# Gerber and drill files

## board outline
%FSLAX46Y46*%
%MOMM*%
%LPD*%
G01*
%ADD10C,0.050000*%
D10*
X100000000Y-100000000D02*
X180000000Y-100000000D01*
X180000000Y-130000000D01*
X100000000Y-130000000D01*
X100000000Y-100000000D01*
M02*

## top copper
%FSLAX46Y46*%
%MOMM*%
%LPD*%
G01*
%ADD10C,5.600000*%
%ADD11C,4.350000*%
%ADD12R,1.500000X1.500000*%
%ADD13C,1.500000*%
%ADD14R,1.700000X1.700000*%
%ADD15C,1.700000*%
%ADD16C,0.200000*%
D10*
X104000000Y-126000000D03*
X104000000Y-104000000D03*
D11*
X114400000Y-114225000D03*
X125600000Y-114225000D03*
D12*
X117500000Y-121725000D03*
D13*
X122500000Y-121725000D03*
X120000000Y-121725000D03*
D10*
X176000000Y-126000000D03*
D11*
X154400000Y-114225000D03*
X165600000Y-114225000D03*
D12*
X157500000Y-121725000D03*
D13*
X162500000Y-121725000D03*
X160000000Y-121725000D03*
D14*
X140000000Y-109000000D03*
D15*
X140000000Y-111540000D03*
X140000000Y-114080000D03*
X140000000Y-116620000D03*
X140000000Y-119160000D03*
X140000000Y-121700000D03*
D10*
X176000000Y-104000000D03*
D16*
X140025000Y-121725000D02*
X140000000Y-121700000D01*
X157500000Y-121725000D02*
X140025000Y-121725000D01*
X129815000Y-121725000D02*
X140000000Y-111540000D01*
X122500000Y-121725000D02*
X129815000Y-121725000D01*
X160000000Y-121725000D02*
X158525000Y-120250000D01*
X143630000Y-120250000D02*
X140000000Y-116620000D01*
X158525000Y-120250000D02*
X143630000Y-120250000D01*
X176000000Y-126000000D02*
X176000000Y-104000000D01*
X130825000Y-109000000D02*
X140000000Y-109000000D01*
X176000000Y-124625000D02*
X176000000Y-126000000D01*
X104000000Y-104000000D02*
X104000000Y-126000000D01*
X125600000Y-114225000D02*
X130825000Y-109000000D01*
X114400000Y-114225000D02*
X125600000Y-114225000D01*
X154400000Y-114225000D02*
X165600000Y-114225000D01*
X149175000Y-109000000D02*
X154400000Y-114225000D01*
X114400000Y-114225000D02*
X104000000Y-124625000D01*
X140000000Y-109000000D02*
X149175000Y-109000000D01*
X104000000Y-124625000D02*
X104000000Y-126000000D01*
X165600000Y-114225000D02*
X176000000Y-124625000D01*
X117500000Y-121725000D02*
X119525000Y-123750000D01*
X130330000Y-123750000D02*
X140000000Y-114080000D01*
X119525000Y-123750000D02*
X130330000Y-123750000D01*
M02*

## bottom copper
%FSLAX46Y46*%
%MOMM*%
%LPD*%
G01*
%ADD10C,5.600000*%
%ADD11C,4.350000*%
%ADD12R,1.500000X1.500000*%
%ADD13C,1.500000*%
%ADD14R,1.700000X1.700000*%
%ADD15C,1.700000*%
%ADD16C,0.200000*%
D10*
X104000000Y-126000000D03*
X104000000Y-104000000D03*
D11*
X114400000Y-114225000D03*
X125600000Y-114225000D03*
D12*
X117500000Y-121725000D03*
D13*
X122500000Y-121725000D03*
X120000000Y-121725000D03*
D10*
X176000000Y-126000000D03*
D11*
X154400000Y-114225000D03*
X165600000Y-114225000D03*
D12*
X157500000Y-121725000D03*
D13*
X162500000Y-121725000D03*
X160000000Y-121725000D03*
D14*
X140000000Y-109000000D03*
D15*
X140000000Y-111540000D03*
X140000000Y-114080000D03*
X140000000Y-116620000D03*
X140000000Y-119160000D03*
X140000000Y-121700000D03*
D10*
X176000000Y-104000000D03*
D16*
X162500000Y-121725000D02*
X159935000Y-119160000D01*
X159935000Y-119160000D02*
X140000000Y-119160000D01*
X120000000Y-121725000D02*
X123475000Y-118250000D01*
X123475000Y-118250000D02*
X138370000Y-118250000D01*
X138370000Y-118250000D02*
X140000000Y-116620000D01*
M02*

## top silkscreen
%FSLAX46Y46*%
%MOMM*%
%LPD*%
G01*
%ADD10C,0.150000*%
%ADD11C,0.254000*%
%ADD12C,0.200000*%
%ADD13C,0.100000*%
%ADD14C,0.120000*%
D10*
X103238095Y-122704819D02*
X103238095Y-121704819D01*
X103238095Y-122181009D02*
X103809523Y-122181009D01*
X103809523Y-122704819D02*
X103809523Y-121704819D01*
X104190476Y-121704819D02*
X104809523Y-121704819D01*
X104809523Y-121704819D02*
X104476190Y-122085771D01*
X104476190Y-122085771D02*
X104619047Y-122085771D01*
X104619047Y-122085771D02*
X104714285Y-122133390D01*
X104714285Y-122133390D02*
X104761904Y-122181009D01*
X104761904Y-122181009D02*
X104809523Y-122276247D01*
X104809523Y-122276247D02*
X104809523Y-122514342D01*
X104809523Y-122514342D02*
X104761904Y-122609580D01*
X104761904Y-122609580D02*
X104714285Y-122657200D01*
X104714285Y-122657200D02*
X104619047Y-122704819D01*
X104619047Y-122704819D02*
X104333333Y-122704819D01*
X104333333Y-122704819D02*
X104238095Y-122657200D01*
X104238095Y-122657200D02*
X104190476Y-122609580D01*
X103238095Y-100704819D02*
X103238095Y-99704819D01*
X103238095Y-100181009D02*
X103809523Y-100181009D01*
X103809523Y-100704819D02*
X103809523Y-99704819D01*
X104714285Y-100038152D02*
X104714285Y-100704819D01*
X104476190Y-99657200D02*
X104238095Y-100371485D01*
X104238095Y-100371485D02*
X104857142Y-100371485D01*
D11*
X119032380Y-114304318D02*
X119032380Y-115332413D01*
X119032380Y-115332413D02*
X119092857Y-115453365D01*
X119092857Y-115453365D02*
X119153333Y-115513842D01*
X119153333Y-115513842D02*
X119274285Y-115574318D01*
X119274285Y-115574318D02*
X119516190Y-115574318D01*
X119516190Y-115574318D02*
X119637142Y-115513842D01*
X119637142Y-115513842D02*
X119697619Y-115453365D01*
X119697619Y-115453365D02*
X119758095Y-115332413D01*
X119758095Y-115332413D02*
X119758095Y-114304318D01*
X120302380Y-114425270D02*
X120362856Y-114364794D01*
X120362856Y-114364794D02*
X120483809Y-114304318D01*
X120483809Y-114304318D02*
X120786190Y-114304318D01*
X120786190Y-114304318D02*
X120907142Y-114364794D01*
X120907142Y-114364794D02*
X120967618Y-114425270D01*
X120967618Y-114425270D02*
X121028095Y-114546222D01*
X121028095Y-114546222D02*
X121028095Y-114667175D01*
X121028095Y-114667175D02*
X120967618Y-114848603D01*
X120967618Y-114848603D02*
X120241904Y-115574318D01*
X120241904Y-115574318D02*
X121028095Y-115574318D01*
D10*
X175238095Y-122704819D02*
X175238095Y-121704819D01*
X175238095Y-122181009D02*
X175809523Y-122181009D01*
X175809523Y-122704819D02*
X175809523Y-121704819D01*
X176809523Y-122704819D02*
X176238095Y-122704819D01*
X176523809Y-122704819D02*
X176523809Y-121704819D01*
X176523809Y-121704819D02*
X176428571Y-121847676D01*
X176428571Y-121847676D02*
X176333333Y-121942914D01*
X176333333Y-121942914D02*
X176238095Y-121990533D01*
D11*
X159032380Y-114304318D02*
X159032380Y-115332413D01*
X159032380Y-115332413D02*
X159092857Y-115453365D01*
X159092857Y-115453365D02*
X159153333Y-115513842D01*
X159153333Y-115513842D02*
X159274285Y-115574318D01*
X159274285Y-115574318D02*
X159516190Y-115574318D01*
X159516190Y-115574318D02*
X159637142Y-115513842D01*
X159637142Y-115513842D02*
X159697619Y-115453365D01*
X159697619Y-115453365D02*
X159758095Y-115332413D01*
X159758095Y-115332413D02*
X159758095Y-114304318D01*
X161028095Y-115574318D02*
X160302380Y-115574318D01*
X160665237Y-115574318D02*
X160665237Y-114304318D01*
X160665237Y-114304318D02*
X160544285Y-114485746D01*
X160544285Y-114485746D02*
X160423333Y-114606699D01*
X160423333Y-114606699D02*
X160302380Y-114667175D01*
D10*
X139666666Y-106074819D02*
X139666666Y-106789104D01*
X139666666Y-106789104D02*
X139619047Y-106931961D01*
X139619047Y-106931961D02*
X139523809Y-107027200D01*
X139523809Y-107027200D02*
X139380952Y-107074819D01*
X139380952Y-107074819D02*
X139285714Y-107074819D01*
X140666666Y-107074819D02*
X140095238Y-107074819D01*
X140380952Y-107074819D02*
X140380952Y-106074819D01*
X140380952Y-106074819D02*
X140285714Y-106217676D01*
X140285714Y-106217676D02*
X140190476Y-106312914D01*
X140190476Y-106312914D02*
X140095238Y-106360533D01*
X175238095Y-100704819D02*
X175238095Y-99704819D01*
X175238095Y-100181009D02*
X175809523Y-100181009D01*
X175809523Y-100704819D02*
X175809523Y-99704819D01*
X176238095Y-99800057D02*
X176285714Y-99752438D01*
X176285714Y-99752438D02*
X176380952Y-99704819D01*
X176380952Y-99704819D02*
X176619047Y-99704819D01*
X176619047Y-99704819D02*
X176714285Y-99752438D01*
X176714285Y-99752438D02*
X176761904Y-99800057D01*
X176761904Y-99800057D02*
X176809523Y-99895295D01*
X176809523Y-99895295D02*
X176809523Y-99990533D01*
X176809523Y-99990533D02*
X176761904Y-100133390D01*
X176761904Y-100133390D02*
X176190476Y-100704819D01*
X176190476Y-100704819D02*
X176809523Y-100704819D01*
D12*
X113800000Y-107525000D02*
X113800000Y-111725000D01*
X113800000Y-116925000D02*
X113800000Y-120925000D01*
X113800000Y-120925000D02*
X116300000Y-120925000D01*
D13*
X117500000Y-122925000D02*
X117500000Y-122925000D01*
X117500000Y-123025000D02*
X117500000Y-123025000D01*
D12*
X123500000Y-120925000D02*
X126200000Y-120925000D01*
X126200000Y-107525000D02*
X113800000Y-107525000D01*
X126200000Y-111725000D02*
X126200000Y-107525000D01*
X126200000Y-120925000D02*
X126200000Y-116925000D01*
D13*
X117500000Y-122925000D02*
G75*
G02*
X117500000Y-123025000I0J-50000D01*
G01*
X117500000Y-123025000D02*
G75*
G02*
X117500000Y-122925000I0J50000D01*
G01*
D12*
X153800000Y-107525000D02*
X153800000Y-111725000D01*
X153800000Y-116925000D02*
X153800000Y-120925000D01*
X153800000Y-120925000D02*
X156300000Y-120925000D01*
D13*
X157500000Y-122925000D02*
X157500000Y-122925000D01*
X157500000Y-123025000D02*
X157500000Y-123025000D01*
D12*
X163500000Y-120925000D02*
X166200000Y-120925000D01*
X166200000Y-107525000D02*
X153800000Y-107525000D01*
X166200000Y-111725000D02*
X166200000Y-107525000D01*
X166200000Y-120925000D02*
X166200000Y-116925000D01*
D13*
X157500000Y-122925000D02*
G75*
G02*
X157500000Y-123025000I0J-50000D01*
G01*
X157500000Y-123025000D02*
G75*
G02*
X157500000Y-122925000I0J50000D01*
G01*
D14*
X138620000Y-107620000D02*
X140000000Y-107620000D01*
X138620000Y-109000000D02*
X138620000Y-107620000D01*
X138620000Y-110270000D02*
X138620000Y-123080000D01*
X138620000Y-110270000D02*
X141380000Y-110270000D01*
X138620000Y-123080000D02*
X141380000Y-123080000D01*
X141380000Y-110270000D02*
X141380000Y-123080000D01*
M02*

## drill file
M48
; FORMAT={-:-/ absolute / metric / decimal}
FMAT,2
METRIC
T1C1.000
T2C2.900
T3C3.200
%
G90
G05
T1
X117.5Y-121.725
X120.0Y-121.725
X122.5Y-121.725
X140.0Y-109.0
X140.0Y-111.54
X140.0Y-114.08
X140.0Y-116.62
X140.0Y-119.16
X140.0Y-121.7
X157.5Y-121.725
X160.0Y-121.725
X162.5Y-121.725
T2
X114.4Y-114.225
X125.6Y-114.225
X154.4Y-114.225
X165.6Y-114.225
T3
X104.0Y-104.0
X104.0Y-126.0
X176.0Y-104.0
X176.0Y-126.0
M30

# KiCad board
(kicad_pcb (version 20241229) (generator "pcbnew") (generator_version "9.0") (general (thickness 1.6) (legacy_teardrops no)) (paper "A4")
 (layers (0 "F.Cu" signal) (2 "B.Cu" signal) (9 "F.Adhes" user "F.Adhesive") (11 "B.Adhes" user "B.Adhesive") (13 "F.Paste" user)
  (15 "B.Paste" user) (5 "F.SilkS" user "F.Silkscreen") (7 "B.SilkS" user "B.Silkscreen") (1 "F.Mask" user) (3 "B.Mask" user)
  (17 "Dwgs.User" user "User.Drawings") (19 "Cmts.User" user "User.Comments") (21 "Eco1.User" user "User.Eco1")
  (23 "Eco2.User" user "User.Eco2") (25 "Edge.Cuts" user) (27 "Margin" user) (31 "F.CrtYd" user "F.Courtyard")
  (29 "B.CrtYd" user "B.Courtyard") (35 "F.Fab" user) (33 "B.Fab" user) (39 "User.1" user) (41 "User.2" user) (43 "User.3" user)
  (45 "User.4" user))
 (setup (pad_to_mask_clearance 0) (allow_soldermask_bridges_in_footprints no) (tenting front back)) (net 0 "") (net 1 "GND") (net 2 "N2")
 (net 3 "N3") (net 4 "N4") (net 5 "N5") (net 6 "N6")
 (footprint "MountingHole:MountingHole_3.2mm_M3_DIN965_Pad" (layer "F.Cu") (at 104 126)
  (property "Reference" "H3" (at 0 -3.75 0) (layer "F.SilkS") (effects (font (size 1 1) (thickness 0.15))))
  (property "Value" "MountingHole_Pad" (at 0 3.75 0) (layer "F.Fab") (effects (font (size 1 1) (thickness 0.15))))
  (pad "1" thru_hole circle (at 0 0) (size 5.6 5.6) (drill 3.2) (layers "*.Cu" "*.Mask") (remove_unused_layers no) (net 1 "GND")
   (zone_connect 2)))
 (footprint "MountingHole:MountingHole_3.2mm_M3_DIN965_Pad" (layer "F.Cu") (at 104 104)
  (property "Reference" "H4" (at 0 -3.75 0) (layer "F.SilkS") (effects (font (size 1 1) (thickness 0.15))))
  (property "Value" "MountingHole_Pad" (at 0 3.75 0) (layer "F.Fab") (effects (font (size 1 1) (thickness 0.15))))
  (pad "1" thru_hole circle (at 0 0) (size 5.6 5.6) (drill 3.2) (layers "*.Cu" "*.Mask") (remove_unused_layers no) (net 1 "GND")
   (zone_connect 2)))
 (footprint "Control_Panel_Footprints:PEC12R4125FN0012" (layer "F.Cu") (at 117.5 121.725)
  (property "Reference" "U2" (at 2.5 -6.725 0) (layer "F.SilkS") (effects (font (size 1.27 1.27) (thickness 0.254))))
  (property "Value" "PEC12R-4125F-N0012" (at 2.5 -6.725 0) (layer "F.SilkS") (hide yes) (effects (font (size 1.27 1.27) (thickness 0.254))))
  (fp_line (start -3.7 -14.2) (end -3.7 -10) (stroke (width 0.2) (type solid)) (layer "F.SilkS"))
  (fp_line (start -3.7 -4.8) (end -3.7 -0.8) (stroke (width 0.2) (type solid)) (layer "F.SilkS"))
  (fp_line (start -3.7 -0.8) (end -1.2 -0.8) (stroke (width 0.2) (type solid)) (layer "F.SilkS"))
  (fp_line (start 0 1.2) (end 0 1.2) (stroke (width 0.1) (type solid)) (layer "F.SilkS"))
  (fp_line (start 0 1.3) (end 0 1.3) (stroke (width 0.1) (type solid)) (layer "F.SilkS"))
  (fp_line (start 6 -0.8) (end 8.7 -0.8) (stroke (width 0.2) (type solid)) (layer "F.SilkS"))
  (fp_line (start 8.7 -14.2) (end -3.7 -14.2) (stroke (width 0.2) (type solid)) (layer "F.SilkS"))
  (fp_line (start 8.7 -10) (end 8.7 -14.2) (stroke (width 0.2) (type solid)) (layer "F.SilkS"))
  (fp_line (start 8.7 -0.8) (end 8.7 -4.8) (stroke (width 0.2) (type solid)) (layer "F.SilkS"))
  (fp_arc (start 0 1.2) (mid 0.05 1.25) (end 0 1.3) (stroke (width 0.1) (type solid)) (layer "F.SilkS"))
  (fp_arc (start 0 1.3) (mid -0.05 1.25) (end 0 1.2) (stroke (width 0.1) (type solid)) (layer "F.SilkS"))
  (pad "1" thru_hole circle (at -3.1 -7.5) (size 4.35 4.35) (drill 2.9) (layers "*.Cu" "*.Mask") (remove_unused_layers no) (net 1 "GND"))
  (pad "2" thru_hole circle (at 8.1 -7.5) (size 4.35 4.35) (drill 2.9) (layers "*.Cu" "*.Mask") (remove_unused_layers no) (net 1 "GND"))
  (pad "A1" thru_hole rect (at 0 0) (size 1.5 1.5) (drill 1) (layers "*.Cu" "*.Mask") (remove_unused_layers no) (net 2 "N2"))
  (pad "B1" thru_hole circle (at 5 0) (size 1.5 1.5) (drill 1) (layers "*.Cu" "*.Mask") (remove_unused_layers no) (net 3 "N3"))
  (pad "C1" thru_hole circle (at 2.5 0) (size 1.5 1.5) (drill 1) (layers "*.Cu" "*.Mask") (remove_unused_layers no) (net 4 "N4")))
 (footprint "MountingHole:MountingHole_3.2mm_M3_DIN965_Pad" (layer "F.Cu") (at 176 126)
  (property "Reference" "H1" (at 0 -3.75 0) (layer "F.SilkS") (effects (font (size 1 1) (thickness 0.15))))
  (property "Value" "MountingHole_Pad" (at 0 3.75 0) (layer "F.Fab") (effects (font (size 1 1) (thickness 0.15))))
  (pad "1" thru_hole circle (at 0 0) (size 5.6 5.6) (drill 3.2) (layers "*.Cu" "*.Mask") (remove_unused_layers no) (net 1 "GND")
   (zone_connect 2)))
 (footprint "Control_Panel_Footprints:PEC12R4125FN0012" (layer "F.Cu") (at 157.5 121.725)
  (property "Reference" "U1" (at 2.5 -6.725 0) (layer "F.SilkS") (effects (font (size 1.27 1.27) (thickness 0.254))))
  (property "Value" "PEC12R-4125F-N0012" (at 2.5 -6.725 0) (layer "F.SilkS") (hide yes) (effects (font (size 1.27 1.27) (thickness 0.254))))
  (fp_line (start -3.7 -14.2) (end -3.7 -10) (stroke (width 0.2) (type solid)) (layer "F.SilkS"))
  (fp_line (start -3.7 -4.8) (end -3.7 -0.8) (stroke (width 0.2) (type solid)) (layer "F.SilkS"))
  (fp_line (start -3.7 -0.8) (end -1.2 -0.8) (stroke (width 0.2) (type solid)) (layer "F.SilkS"))
  (fp_line (start 0 1.2) (end 0 1.2) (stroke (width 0.1) (type solid)) (layer "F.SilkS"))
  (fp_line (start 0 1.3) (end 0 1.3) (stroke (width 0.1) (type solid)) (layer "F.SilkS"))
  (fp_line (start 6 -0.8) (end 8.7 -0.8) (stroke (width 0.2) (type solid)) (layer "F.SilkS"))
  (fp_line (start 8.7 -14.2) (end -3.7 -14.2) (stroke (width 0.2) (type solid)) (layer "F.SilkS"))
  (fp_line (start 8.7 -10) (end 8.7 -14.2) (stroke (width 0.2) (type solid)) (layer "F.SilkS"))
  (fp_line (start 8.7 -0.8) (end 8.7 -4.8) (stroke (width 0.2) (type solid)) (layer "F.SilkS"))
  (fp_arc (start 0 1.2) (mid 0.05 1.25) (end 0 1.3) (stroke (width 0.1) (type solid)) (layer "F.SilkS"))
  (fp_arc (start 0 1.3) (mid -0.05 1.25) (end 0 1.2) (stroke (width 0.1) (type solid)) (layer "F.SilkS"))
  (pad "1" thru_hole circle (at -3.1 -7.5) (size 4.35 4.35) (drill 2.9) (layers "*.Cu" "*.Mask") (remove_unused_layers no) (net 1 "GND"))
  (pad "2" thru_hole circle (at 8.1 -7.5) (size 4.35 4.35) (drill 2.9) (layers "*.Cu" "*.Mask") (remove_unused_layers no) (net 1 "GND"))
  (pad "A1" thru_hole rect (at 0 0) (size 1.5 1.5) (drill 1) (layers "*.Cu" "*.Mask") (remove_unused_layers no) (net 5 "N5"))
  (pad "B1" thru_hole circle (at 5 0) (size 1.5 1.5) (drill 1) (layers "*.Cu" "*.Mask") (remove_unused_layers no) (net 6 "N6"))
  (pad "C1" thru_hole circle (at 2.5 0) (size 1.5 1.5) (drill 1) (layers "*.Cu" "*.Mask") (remove_unused_layers no) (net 4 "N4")))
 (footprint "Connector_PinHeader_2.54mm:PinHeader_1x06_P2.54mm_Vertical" (layer "F.Cu") (at 140 109)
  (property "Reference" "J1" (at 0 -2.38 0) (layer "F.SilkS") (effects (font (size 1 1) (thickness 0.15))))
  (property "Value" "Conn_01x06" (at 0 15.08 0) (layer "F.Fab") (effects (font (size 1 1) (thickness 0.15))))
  (fp_line (start -1.38 -1.38) (end 0 -1.38) (stroke (width 0.12) (type solid)) (layer "F.SilkS"))
  (fp_line (start -1.38 0) (end -1.38 -1.38) (stroke (width 0.12) (type solid)) (layer "F.SilkS"))
  (fp_line (start -1.38 1.27) (end -1.38 14.08) (stroke (width 0.12) (type solid)) (layer "F.SilkS"))
  (fp_line (start -1.38 1.27) (end 1.38 1.27) (stroke (width 0.12) (type solid)) (layer "F.SilkS"))
  (fp_line (start -1.38 14.08) (end 1.38 14.08) (stroke (width 0.12) (type solid)) (layer "F.SilkS"))
  (fp_line (start 1.38 1.27) (end 1.38 14.08) (stroke (width 0.12) (type solid)) (layer "F.SilkS"))
  (pad "1" thru_hole rect (at 0 0) (size 1.7 1.7) (drill 1) (layers "*.Cu" "*.Mask") (remove_unused_layers no) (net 1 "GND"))
  (pad "2" thru_hole circle (at 0 2.54) (size 1.7 1.7) (drill 1) (layers "*.Cu" "*.Mask") (remove_unused_layers no) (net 3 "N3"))
  (pad "3" thru_hole circle (at 0 5.08) (size 1.7 1.7) (drill 1) (layers "*.Cu" "*.Mask") (remove_unused_layers no) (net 2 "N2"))
  (pad "4" thru_hole circle (at 0 7.62) (size 1.7 1.7) (drill 1) (layers "*.Cu" "*.Mask") (remove_unused_layers no) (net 4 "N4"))
  (pad "5" thru_hole circle (at 0 10.16) (size 1.7 1.7) (drill 1) (layers "*.Cu" "*.Mask") (remove_unused_layers no) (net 6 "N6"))
  (pad "6" thru_hole circle (at 0 12.7) (size 1.7 1.7) (drill 1) (layers "*.Cu" "*.Mask") (remove_unused_layers no) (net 5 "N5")))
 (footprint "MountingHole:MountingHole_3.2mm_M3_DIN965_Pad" (layer "F.Cu") (at 176 104)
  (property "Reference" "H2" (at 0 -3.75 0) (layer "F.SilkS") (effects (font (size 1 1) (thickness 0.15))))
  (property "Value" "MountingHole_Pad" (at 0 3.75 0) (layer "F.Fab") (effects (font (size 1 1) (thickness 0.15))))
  (pad "1" thru_hole circle (at 0 0) (size 5.6 5.6) (drill 3.2) (layers "*.Cu" "*.Mask") (remove_unused_layers no) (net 1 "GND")
   (zone_connect 2)))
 (gr_rect (start 100 100) (end 180 130) (stroke (width 0.05) (type solid)) (fill no) (layer "Edge.Cuts"))
 (segment (start 140.025 121.725) (end 140 121.7) (width 0.2) (layer "F.Cu") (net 5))
 (segment (start 157.5 121.725) (end 140.025 121.725) (width 0.2) (layer "F.Cu") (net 5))
 (segment (start 162.5 121.725) (end 159.935 119.16) (width 0.2) (layer "B.Cu") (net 6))
 (segment (start 159.935 119.16) (end 140 119.16) (width 0.2) (layer "B.Cu") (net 6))
 (segment (start 129.815 121.725) (end 140 111.54) (width 0.2) (layer "F.Cu") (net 3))
 (segment (start 122.5 121.725) (end 129.815 121.725) (width 0.2) (layer "F.Cu") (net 3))
 (segment (start 160 121.725) (end 158.525 120.25) (width 0.2) (layer "F.Cu") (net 4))
 (segment (start 143.63 120.25) (end 140 116.62) (width 0.2) (layer "F.Cu") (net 4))
 (segment (start 158.525 120.25) (end 143.63 120.25) (width 0.2) (layer "F.Cu") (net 4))
 (segment (start 120 121.725) (end 123.475 118.25) (width 0.2) (layer "B.Cu") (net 4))
 (segment (start 123.475 118.25) (end 138.37 118.25) (width 0.2) (layer "B.Cu") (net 4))
 (segment (start 138.37 118.25) (end 140 116.62) (width 0.2) (layer "B.Cu") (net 4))
 (segment (start 176 126) (end 176 104) (width 0.2) (layer "F.Cu") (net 1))
 (segment (start 130.825 109) (end 140 109) (width 0.2) (layer "F.Cu") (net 1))
 (segment (start 176 124.625) (end 176 126) (width 0.2) (layer "F.Cu") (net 1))
 (segment (start 104 104) (end 104 126) (width 0.2) (layer "F.Cu") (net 1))
 (segment (start 125.6 114.225) (end 130.825 109) (width 0.2) (layer "F.Cu") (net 1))
 (segment (start 114.4 114.225) (end 125.6 114.225) (width 0.2) (layer "F.Cu") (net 1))
 (segment (start 154.4 114.225) (end 165.6 114.225) (width 0.2) (layer "F.Cu") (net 1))
 (segment (start 149.175 109) (end 154.4 114.225) (width 0.2) (layer "F.Cu") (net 1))
 (segment (start 114.4 114.225) (end 104 124.625) (width 0.2) (layer "F.Cu") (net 1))
 (segment (start 140 109) (end 149.175 109) (width 0.2) (layer "F.Cu") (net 1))
 (segment (start 104 124.625) (end 104 126) (width 0.2) (layer "F.Cu") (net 1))
 (segment (start 165.6 114.225) (end 176 124.625) (width 0.2) (layer "F.Cu") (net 1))
 (segment (start 117.5 121.725) (end 119.525 123.75) (width 0.2) (layer "F.Cu") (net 2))
 (segment (start 130.33 123.75) (end 140 114.08) (width 0.2) (layer "F.Cu") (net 2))
 (segment (start 119.525 123.75) (end 130.33 123.75) (width 0.2) (layer "F.Cu") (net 2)))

